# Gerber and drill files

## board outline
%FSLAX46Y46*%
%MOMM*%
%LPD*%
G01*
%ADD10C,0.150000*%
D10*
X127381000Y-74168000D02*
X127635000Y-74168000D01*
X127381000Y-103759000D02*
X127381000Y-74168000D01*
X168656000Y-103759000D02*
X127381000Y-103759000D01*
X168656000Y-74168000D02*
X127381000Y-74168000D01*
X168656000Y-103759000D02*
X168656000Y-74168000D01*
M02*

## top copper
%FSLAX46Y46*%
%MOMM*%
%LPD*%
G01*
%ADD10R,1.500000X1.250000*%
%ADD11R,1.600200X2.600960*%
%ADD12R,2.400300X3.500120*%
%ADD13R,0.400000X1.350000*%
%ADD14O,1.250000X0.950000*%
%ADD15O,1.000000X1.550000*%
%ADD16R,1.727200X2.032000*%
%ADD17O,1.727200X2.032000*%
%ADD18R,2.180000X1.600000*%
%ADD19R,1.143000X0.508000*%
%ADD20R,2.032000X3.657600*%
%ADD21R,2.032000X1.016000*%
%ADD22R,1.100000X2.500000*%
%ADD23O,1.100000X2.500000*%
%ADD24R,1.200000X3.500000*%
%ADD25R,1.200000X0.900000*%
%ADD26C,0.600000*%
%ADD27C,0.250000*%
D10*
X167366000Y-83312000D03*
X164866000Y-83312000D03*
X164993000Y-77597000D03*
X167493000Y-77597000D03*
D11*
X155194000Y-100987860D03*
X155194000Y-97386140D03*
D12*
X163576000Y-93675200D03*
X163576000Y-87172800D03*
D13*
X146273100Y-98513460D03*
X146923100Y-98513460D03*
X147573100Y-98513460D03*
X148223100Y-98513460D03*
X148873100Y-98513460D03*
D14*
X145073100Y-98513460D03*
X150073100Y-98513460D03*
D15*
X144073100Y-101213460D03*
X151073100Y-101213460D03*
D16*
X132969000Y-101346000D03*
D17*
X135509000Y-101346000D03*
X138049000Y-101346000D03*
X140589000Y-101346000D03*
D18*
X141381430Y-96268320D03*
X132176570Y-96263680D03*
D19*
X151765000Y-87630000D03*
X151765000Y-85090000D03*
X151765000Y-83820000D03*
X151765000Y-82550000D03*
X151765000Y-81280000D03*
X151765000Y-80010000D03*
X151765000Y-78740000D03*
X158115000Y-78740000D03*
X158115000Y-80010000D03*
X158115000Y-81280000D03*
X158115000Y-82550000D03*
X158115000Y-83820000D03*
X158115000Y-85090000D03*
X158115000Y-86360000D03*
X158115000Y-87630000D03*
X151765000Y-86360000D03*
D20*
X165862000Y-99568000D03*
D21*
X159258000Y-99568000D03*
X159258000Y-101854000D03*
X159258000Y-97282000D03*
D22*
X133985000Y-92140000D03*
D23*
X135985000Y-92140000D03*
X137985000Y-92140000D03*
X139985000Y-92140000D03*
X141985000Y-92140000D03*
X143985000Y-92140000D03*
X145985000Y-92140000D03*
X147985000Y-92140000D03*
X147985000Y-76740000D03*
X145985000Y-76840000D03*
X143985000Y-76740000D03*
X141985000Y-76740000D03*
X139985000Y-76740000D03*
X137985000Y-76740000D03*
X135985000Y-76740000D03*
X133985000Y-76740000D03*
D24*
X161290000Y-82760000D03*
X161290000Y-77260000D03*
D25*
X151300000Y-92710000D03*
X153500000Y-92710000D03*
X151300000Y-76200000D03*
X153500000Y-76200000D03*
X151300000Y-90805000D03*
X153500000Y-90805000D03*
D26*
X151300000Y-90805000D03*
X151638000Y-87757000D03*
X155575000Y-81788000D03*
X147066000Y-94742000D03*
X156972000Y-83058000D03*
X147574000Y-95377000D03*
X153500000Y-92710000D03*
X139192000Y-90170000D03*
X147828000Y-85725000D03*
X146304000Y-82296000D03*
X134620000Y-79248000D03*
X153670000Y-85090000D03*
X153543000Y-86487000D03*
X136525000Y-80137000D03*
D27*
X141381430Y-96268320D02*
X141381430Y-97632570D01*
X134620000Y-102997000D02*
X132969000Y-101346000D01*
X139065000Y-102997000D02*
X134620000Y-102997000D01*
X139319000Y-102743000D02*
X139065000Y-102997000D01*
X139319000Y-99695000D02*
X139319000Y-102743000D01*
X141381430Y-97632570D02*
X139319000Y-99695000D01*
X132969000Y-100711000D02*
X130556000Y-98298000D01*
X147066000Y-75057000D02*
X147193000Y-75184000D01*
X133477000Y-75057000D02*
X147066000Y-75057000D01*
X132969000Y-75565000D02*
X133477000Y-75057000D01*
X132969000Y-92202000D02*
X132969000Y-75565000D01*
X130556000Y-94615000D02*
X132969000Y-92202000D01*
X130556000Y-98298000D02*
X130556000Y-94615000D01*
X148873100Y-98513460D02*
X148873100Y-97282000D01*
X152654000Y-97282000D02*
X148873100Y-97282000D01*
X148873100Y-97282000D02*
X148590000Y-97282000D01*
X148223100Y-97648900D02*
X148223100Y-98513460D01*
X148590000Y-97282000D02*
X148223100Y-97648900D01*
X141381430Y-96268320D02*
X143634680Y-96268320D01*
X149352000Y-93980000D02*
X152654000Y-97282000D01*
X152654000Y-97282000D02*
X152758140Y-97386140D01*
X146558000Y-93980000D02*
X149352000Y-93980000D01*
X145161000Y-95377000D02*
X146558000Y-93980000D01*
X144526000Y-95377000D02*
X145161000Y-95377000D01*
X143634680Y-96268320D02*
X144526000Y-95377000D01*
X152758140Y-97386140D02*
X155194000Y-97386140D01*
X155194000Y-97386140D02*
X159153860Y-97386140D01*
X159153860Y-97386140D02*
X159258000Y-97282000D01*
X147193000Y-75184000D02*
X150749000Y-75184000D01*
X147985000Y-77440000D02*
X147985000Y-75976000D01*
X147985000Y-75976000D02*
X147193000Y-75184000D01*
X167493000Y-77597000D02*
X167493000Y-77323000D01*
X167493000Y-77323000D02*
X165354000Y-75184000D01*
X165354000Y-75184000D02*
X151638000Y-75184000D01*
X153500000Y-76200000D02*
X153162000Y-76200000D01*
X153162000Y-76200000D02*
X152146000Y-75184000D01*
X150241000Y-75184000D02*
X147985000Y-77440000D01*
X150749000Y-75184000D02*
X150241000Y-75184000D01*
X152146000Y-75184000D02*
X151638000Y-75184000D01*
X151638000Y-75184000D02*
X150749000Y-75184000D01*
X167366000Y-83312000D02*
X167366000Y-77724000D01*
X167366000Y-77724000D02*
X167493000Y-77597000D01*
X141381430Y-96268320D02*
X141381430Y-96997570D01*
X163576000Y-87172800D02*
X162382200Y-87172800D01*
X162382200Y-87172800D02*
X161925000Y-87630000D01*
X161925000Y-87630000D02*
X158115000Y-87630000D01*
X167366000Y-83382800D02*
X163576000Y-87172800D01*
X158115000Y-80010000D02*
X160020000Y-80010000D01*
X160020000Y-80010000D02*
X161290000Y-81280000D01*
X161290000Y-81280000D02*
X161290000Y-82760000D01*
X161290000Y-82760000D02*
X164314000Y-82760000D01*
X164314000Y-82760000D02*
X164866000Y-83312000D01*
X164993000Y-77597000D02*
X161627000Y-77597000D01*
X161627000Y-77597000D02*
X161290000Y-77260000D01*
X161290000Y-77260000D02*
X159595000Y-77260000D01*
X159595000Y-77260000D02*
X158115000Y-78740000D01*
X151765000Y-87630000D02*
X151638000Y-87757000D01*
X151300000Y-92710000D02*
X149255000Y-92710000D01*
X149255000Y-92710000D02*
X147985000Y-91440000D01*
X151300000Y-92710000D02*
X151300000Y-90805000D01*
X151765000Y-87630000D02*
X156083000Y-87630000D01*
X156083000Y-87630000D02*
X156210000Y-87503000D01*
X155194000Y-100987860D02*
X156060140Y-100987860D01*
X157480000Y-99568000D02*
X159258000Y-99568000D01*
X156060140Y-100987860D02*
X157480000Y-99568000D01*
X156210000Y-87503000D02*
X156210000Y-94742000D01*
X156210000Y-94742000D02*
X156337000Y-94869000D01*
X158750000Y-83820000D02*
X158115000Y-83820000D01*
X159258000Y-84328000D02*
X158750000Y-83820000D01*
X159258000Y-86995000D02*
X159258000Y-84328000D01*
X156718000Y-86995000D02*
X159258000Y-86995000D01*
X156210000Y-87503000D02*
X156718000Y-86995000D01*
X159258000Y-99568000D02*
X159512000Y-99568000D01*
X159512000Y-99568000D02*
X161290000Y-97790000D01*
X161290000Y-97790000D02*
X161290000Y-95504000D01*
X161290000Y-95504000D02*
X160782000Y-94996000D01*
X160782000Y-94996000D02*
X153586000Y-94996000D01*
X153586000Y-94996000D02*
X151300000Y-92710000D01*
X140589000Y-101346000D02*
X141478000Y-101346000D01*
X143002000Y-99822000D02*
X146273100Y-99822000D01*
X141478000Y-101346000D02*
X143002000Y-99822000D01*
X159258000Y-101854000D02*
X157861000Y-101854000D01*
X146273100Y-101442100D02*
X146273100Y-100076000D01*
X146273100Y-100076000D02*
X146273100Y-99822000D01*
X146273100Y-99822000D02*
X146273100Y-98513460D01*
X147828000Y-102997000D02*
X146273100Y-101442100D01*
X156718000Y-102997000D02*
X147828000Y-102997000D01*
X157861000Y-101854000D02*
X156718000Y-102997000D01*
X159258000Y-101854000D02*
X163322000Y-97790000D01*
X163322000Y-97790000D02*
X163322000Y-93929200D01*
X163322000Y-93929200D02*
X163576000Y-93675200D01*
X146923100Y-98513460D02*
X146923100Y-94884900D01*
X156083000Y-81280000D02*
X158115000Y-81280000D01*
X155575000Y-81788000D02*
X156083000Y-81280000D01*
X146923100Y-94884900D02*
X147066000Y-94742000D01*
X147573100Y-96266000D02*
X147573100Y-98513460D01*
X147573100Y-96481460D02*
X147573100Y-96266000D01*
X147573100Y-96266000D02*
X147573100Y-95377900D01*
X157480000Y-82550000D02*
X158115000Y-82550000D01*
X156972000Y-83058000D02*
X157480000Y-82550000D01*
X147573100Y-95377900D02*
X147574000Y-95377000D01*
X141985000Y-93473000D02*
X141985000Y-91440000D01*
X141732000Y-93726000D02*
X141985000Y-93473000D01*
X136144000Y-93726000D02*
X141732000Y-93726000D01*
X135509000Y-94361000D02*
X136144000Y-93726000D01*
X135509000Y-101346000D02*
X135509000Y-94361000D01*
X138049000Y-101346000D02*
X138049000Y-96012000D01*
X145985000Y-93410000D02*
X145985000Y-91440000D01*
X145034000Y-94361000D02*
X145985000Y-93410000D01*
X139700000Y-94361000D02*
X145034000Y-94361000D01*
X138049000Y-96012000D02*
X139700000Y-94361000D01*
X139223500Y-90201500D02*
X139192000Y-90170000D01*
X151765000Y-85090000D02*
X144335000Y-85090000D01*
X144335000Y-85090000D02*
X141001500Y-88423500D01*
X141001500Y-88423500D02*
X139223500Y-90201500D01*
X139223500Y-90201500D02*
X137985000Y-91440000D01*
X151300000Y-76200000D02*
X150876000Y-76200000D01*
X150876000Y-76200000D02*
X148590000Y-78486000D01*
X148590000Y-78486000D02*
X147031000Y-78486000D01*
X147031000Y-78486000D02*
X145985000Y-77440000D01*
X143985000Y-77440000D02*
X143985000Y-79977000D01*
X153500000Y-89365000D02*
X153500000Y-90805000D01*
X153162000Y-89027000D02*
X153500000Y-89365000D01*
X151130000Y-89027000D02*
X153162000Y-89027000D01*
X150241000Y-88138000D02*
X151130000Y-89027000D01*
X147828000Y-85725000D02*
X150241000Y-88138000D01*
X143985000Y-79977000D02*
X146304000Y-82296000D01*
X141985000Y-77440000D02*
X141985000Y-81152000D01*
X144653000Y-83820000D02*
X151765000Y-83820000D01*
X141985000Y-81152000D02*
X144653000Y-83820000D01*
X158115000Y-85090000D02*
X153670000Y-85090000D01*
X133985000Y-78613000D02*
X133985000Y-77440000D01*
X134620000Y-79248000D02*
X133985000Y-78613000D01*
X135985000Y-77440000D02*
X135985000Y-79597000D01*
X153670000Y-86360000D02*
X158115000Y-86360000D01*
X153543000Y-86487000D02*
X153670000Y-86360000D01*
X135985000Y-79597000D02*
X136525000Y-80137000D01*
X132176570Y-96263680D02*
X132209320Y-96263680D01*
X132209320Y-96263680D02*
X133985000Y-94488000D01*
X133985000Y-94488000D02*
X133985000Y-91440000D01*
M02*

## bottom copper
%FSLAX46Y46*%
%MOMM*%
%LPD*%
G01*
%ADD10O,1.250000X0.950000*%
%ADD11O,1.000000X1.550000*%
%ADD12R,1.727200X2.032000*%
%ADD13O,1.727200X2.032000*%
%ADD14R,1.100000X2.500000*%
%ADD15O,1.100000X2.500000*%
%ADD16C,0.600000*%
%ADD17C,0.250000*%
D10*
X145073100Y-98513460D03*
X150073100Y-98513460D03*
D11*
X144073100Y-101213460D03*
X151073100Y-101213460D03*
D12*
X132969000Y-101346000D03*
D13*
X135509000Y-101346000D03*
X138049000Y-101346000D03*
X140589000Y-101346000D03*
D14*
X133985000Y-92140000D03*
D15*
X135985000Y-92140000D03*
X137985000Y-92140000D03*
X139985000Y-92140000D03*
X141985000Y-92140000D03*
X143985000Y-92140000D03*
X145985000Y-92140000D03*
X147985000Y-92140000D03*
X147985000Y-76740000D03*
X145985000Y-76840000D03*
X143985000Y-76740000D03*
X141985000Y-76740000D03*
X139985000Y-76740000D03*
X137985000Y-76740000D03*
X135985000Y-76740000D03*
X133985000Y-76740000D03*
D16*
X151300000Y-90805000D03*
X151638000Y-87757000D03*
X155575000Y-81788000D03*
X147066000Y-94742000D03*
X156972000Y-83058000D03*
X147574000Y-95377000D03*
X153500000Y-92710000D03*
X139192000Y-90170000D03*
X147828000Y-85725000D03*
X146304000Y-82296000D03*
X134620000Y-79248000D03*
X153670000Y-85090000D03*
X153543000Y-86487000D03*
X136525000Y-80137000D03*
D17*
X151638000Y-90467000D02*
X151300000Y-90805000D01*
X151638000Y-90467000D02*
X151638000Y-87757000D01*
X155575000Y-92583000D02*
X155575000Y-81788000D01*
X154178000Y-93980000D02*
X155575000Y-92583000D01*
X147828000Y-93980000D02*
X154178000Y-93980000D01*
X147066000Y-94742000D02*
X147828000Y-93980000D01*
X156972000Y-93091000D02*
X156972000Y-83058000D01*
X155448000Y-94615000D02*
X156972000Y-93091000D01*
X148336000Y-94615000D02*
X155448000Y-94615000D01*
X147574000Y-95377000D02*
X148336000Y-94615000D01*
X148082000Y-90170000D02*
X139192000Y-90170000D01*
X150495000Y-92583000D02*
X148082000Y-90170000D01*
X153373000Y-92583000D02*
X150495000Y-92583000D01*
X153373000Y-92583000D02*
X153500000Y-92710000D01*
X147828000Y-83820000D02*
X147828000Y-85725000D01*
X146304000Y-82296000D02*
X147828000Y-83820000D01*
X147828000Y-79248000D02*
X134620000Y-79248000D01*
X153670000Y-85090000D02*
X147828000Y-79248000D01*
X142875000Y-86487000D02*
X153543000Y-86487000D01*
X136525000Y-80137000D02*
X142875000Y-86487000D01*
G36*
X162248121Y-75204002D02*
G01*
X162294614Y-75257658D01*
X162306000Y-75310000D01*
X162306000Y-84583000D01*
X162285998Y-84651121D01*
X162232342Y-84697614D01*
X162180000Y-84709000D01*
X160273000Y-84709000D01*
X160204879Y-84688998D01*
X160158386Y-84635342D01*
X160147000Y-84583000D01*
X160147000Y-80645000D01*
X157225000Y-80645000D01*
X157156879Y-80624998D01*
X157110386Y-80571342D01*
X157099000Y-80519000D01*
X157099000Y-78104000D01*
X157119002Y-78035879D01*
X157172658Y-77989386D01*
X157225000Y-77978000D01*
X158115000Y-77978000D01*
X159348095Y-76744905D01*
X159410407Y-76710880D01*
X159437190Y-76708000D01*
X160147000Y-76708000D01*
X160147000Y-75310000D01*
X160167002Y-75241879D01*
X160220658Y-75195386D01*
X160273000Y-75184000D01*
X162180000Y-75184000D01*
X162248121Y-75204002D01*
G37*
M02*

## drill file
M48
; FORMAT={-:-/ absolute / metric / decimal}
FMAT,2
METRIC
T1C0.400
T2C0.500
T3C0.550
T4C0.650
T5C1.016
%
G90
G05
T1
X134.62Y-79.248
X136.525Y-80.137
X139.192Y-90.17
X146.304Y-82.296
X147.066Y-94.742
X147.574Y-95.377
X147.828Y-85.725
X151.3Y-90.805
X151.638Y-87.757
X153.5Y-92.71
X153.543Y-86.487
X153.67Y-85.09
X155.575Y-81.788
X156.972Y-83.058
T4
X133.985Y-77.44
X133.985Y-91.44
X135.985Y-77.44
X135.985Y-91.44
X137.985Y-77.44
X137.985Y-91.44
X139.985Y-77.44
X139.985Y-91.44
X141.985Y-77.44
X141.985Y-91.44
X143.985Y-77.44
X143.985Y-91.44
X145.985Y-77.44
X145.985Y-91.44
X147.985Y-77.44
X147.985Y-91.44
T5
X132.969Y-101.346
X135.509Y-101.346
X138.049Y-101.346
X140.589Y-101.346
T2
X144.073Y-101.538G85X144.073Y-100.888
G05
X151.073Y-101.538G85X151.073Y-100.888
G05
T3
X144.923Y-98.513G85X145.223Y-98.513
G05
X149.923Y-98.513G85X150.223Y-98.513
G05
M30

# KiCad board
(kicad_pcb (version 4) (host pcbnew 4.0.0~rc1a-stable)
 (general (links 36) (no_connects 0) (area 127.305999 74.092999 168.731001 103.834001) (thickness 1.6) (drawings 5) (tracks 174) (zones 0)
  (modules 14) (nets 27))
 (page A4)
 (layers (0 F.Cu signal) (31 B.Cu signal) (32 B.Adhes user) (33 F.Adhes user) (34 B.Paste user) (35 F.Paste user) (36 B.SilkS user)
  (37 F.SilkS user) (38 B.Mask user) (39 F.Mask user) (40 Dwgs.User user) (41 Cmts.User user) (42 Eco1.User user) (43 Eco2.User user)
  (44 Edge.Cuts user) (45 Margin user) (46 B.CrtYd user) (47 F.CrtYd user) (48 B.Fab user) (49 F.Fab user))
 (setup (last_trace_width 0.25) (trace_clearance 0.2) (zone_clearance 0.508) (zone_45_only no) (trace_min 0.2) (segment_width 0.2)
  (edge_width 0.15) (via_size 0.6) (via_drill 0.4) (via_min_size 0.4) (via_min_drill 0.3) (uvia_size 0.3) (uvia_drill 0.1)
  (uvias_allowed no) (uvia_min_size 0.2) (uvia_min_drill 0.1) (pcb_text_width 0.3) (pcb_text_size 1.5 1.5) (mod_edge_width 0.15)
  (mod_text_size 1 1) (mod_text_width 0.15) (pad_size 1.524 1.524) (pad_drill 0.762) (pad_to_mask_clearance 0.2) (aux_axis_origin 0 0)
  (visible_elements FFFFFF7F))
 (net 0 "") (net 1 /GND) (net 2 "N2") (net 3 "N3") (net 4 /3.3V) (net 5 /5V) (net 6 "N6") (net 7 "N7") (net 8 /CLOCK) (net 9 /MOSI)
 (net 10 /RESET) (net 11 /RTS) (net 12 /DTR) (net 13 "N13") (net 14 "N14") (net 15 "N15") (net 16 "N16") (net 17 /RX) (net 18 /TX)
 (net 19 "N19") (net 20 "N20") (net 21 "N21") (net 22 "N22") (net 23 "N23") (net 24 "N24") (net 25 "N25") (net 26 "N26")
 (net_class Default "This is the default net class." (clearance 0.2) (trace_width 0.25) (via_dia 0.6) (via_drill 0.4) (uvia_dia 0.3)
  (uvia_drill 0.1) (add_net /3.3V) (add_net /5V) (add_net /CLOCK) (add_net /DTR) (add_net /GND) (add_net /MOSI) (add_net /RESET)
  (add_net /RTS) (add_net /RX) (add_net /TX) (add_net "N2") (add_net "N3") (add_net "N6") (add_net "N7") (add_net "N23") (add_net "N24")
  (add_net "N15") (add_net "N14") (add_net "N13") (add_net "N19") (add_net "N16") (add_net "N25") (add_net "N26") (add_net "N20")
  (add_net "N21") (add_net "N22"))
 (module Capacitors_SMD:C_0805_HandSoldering (layer F.Cu) (at 166.116 83.312 180)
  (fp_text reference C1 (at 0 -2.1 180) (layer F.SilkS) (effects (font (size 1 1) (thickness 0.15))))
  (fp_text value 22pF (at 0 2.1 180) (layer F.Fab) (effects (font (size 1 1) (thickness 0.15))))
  (pad 1 smd rect (at -1.25 0 180) (size 1.5 1.25) (layers F.Cu F.Paste F.Mask) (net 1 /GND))
  (pad 2 smd rect (at 1.25 0 180) (size 1.5 1.25) (layers F.Cu F.Paste F.Mask) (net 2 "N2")))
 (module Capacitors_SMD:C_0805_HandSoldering (layer F.Cu) (at 166.243 77.597)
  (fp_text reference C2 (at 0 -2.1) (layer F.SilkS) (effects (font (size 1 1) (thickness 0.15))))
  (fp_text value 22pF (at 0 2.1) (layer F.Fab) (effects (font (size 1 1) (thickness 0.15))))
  (pad 1 smd rect (at -1.25 0) (size 1.5 1.25) (layers F.Cu F.Paste F.Mask) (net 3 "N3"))
  (pad 2 smd rect (at 1.25 0) (size 1.5 1.25) (layers F.Cu F.Paste F.Mask) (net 1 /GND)))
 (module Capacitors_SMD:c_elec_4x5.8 (layer F.Cu) (at 155.194 99.187 270)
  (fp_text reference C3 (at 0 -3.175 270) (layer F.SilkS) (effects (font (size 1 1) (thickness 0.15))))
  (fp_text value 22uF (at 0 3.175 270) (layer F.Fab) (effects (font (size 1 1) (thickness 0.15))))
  (pad 1 smd rect (at 1.80086 0 270) (size 2.60096 1.6002) (layers F.Cu F.Paste F.Mask) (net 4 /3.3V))
  (pad 2 smd rect (at -1.80086 0 270) (size 2.60096 1.6002) (layers F.Cu F.Paste F.Mask) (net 1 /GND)))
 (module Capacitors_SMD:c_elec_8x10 (layer F.Cu) (at 163.576 90.424 270)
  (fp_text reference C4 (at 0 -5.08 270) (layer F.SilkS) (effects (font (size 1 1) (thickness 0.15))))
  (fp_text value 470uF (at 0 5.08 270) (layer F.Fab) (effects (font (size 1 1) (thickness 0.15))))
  (pad 1 smd rect (at 3.2512 0 270) (size 3.50012 2.4003) (layers F.Cu F.Paste F.Mask) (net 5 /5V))
  (pad 2 smd rect (at -3.2512 0 270) (size 3.50012 2.4003) (layers F.Cu F.Paste F.Mask) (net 1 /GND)))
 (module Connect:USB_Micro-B (layer F.Cu) (at 147.574 100.076)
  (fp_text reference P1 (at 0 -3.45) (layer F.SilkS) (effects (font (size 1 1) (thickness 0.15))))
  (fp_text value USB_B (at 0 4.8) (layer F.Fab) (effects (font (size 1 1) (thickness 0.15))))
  (pad 1 smd rect (at -1.3009 -1.56254 90) (size 1.35 0.4) (layers F.Cu F.Paste F.Mask) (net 5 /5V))
  (pad 2 smd rect (at -0.6509 -1.56254 90) (size 1.35 0.4) (layers F.Cu F.Paste F.Mask) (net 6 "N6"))
  (pad 3 smd rect (at -0.0009 -1.56254 90) (size 1.35 0.4) (layers F.Cu F.Paste F.Mask) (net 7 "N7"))
  (pad 4 smd rect (at 0.6491 -1.56254 90) (size 1.35 0.4) (layers F.Cu F.Paste F.Mask) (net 1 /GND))
  (pad 5 smd rect (at 1.2991 -1.56254 90) (size 1.35 0.4) (layers F.Cu F.Paste F.Mask) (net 1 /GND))
  (pad 6 thru_hole oval (at -2.5009 -1.56254 90) (size 0.95 1.25) (drill oval 0.55 0.85) (layers *.Cu *.Mask F.SilkS))
  (pad 6 thru_hole oval (at 2.4991 -1.56254 90) (size 0.95 1.25) (drill oval 0.55 0.85) (layers *.Cu *.Mask F.SilkS))
  (pad 6 thru_hole oval (at -3.5009 1.13746 90) (size 1.55 1) (drill oval 1.15 0.5) (layers *.Cu *.Mask F.SilkS))
  (pad 6 thru_hole oval (at 3.4991 1.13746 90) (size 1.55 1) (drill oval 1.15 0.5) (layers *.Cu *.Mask F.SilkS)))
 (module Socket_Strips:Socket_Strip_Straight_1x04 (layer F.Cu) (at 132.969 101.346)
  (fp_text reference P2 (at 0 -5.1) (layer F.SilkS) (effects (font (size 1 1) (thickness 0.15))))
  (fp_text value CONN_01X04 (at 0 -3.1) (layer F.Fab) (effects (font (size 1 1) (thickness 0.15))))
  (pad 1 thru_hole rect (at 0 0) (size 1.7272 2.032) (drill 1.016) (layers *.Cu *.Mask F.SilkS) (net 1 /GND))
  (pad 2 thru_hole oval (at 2.54 0) (size 1.7272 2.032) (drill 1.016) (layers *.Cu *.Mask F.SilkS) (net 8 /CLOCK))
  (pad 3 thru_hole oval (at 5.08 0) (size 1.7272 2.032) (drill 1.016) (layers *.Cu *.Mask F.SilkS) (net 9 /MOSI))
  (pad 4 thru_hole oval (at 7.62 0) (size 1.7272 2.032) (drill 1.016) (layers *.Cu *.Mask F.SilkS) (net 5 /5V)))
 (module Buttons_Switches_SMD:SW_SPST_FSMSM (layer F.Cu) (at 136.779 96.266 180)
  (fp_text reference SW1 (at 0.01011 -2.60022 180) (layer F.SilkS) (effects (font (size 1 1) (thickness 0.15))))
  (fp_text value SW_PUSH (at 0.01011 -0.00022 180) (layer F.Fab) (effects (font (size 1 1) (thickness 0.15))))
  (pad 1 smd rect (at -4.60243 -0.00232 180) (size 2.18 1.6) (layers F.Cu F.Paste F.Mask) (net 1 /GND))
  (pad 2 smd rect (at 4.60243 0.00232 180) (size 2.18 1.6) (layers F.Cu F.Paste F.Mask) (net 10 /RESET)))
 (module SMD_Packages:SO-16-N (layer F.Cu) (at 154.94 83.185 90)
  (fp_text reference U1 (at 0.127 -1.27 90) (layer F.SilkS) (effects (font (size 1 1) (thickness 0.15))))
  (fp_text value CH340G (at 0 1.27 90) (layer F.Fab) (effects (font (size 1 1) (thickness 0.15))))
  (pad 16 smd rect (at -4.445 -3.175 90) (size 0.508 1.143) (layers F.Cu F.Paste F.Mask) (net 4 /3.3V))
  (pad 14 smd rect (at -1.905 -3.175 90) (size 0.508 1.143) (layers F.Cu F.Paste F.Mask) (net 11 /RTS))
  (pad 13 smd rect (at -0.635 -3.175 90) (size 0.508 1.143) (layers F.Cu F.Paste F.Mask) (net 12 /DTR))
  (pad 12 smd rect (at 0.635 -3.175 90) (size 0.508 1.143) (layers F.Cu F.Paste F.Mask) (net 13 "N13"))
  (pad 11 smd rect (at 1.905 -3.175 90) (size 0.508 1.143) (layers F.Cu F.Paste F.Mask) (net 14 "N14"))
  (pad 10 smd rect (at 3.175 -3.175 90) (size 0.508 1.143) (layers F.Cu F.Paste F.Mask) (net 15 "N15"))
  (pad 9 smd rect (at 4.445 -3.175 90) (size 0.508 1.143) (layers F.Cu F.Paste F.Mask) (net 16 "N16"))
  (pad 8 smd rect (at 4.445 3.175 90) (size 0.508 1.143) (layers F.Cu F.Paste F.Mask) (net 3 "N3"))
  (pad 7 smd rect (at 3.175 3.175 90) (size 0.508 1.143) (layers F.Cu F.Paste F.Mask) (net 2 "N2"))
  (pad 6 smd rect (at 1.905 3.175 90) (size 0.508 1.143) (layers F.Cu F.Paste F.Mask) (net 6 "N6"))
  (pad 5 smd rect (at 0.635 3.175 90) (size 0.508 1.143) (layers F.Cu F.Paste F.Mask) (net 7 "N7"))
  (pad 4 smd rect (at -0.635 3.175 90) (size 0.508 1.143) (layers F.Cu F.Paste F.Mask) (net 4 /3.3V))
  (pad 3 smd rect (at -1.905 3.175 90) (size 0.508 1.143) (layers F.Cu F.Paste F.Mask) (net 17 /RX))
  (pad 2 smd rect (at -3.175 3.175 90) (size 0.508 1.143) (layers F.Cu F.Paste F.Mask) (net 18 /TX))
  (pad 1 smd rect (at -4.445 3.175 90) (size 0.508 1.143) (layers F.Cu F.Paste F.Mask) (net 1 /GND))
  (pad 15 smd rect (at -3.175 -3.175 90) (size 0.508 1.143) (layers F.Cu F.Paste F.Mask) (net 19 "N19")))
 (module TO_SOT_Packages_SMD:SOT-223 (layer F.Cu) (at 162.56 99.568 270)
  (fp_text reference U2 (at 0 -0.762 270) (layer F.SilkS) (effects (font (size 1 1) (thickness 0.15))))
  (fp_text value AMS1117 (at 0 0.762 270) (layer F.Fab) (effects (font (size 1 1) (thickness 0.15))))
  (pad 4 smd rect (at 0 -3.302 270) (size 3.6576 2.032) (layers F.Cu F.Paste F.Mask))
  (pad 2 smd rect (at 0 3.302 270) (size 1.016 2.032) (layers F.Cu F.Paste F.Mask) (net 4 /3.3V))
  (pad 3 smd rect (at 2.286 3.302 270) (size 1.016 2.032) (layers F.Cu F.Paste F.Mask) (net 5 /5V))
  (pad 1 smd rect (at -2.286 3.302 270) (size 1.016 2.032) (layers F.Cu F.Paste F.Mask) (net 1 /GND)))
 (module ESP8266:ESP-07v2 (layer F.Cu) (at 133.985 91.44 90)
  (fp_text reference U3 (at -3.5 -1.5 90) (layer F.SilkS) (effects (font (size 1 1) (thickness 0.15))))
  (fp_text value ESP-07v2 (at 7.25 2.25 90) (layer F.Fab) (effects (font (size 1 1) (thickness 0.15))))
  (pad 1 thru_hole rect (at 0 0 90) (size 2.5 1.1) (drill 0.65 (offset -0.7 0)) (layers *.Cu *.Mask F.SilkS) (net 10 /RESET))
  (pad 2 thru_hole oval (at 0 2 90) (size 2.5 1.1) (drill 0.65 (offset -0.7 0)) (layers *.Cu *.Mask F.SilkS) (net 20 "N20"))
  (pad 3 thru_hole oval (at 0 4 90) (size 2.5 1.1) (drill 0.65 (offset -0.7 0)) (layers *.Cu *.Mask F.SilkS) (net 11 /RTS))
  (pad 4 thru_hole oval (at 0 6 90) (size 2.5 1.1) (drill 0.65 (offset -0.7 0)) (layers *.Cu *.Mask F.SilkS) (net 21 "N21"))
  (pad 5 thru_hole oval (at 0 8 90) (size 2.5 1.1) (drill 0.65 (offset -0.7 0)) (layers *.Cu *.Mask F.SilkS) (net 8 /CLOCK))
  (pad 6 thru_hole oval (at 0 10 90) (size 2.5 1.1) (drill 0.65 (offset -0.7 0)) (layers *.Cu *.Mask F.SilkS) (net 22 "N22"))
  (pad 7 thru_hole oval (at 0 12 90) (size 2.5 1.1) (drill 0.65 (offset -0.7 0)) (layers *.Cu *.Mask F.SilkS) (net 9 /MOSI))
  (pad 8 thru_hole oval (at 0 14 90) (size 2.5 1.1) (drill 0.65 (offset -0.7 0)) (layers *.Cu *.Mask F.SilkS) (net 4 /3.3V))
  (pad 9 thru_hole oval (at 14 14 90) (size 2.5 1.1) (drill 0.65 (offset 0.7 0)) (layers *.Cu *.Mask F.SilkS) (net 1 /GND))
  (pad 10 thru_hole oval (at 14 12 90) (size 2.5 1.1) (drill 0.65 (offset 0.6 0)) (layers *.Cu *.Mask F.SilkS) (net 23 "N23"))
  (pad 11 thru_hole oval (at 14 10 90) (size 2.5 1.1) (drill 0.65 (offset 0.7 0)) (layers *.Cu *.Mask F.SilkS) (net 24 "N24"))
  (pad 12 thru_hole oval (at 14 8 90) (size 2.5 1.1) (drill 0.65 (offset 0.7 0)) (layers *.Cu *.Mask F.SilkS) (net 12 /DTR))
  (pad 13 thru_hole oval (at 14 6 90) (size 2.5 1.1) (drill 0.65 (offset 0.7 0)) (layers *.Cu *.Mask F.SilkS) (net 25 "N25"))
  (pad 14 thru_hole oval (at 14 4 90) (size 2.5 1.1) (drill 0.65 (offset 0.7 0)) (layers *.Cu *.Mask F.SilkS) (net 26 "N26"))
  (pad 15 thru_hole oval (at 14 2 90) (size 2.5 1.1) (drill 0.65 (offset 0.7 0)) (layers *.Cu *.Mask F.SilkS) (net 18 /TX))
  (pad 16 thru_hole oval (at 14 0 90) (size 2.5 1.1) (drill 0.65 (offset 0.7 0)) (layers *.Cu *.Mask F.SilkS) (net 17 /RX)))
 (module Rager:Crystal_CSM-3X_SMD (layer F.Cu) (at 161.29 80.01 90)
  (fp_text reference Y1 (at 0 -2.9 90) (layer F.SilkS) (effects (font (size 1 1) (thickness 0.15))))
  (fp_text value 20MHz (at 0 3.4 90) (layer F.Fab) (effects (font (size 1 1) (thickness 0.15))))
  (pad 1 smd rect (at -2.75 0 90) (size 3.5 1.2) (layers F.Cu F.Paste F.Mask) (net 2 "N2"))
  (pad 2 smd rect (at 2.75 0 90) (size 3.5 1.2) (layers F.Cu F.Paste F.Mask) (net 3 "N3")))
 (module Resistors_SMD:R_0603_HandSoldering (layer F.Cu) (at 152.4 92.71)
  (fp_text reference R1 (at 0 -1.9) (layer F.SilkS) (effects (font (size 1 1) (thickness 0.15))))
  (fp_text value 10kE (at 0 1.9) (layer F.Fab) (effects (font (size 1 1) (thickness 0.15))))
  (pad 1 smd rect (at -1.1 0) (size 1.2 0.9) (layers F.Cu F.Paste F.Mask) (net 4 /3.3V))
  (pad 2 smd rect (at 1.1 0) (size 1.2 0.9) (layers F.Cu F.Paste F.Mask) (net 11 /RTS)))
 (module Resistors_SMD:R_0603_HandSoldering (layer F.Cu) (at 152.4 76.2)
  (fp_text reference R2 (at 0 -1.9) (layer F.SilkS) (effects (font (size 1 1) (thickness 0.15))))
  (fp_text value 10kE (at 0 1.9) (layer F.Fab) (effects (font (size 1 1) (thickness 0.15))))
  (pad 1 smd rect (at -1.1 0) (size 1.2 0.9) (layers F.Cu F.Paste F.Mask) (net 23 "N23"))
  (pad 2 smd rect (at 1.1 0) (size 1.2 0.9) (layers F.Cu F.Paste F.Mask) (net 1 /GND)))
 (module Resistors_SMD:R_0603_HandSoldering (layer F.Cu) (at 152.4 90.805)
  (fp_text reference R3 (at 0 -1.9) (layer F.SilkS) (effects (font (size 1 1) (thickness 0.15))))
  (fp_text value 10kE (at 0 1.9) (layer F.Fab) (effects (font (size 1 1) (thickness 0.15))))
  (pad 1 smd rect (at -1.1 0) (size 1.2 0.9) (layers F.Cu F.Paste F.Mask) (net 4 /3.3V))
  (pad 2 smd rect (at 1.1 0) (size 1.2 0.9) (layers F.Cu F.Paste F.Mask) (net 24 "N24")))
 (gr_line (start 127.381 74.168) (end 127.635 74.168) (angle 90) (layer Edge.Cuts) (width 0.15))
 (gr_line (start 127.381 103.759) (end 127.381 74.168) (angle 90) (layer Edge.Cuts) (width 0.15))
 (gr_line (start 168.656 103.759) (end 127.381 103.759) (angle 90) (layer Edge.Cuts) (width 0.15))
 (gr_line (start 168.656 74.168) (end 127.381 74.168) (angle 90) (layer Edge.Cuts) (width 0.15))
 (gr_line (start 168.656 103.759) (end 168.656 74.168) (angle 90) (layer Edge.Cuts) (width 0.15))
 (segment (start 141.38143 96.26832) (end 141.38143 97.63257) (width 0.25) (layer F.Cu) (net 1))
 (segment (start 134.62 102.997) (end 132.969 101.346) (width 0.25) (layer F.Cu) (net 1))
 (segment (start 139.065 102.997) (end 134.62 102.997) (width 0.25) (layer F.Cu) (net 1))
 (segment (start 139.319 102.743) (end 139.065 102.997) (width 0.25) (layer F.Cu) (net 1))
 (segment (start 139.319 99.695) (end 139.319 102.743) (width 0.25) (layer F.Cu) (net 1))
 (segment (start 141.38143 97.63257) (end 139.319 99.695) (width 0.25) (layer F.Cu) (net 1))
 (segment (start 132.969 100.711) (end 130.556 98.298) (width 0.25) (layer F.Cu) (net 1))
 (segment (start 147.066 75.057) (end 147.193 75.184) (width 0.25) (layer F.Cu) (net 1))
 (segment (start 133.477 75.057) (end 147.066 75.057) (width 0.25) (layer F.Cu) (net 1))
 (segment (start 132.969 75.565) (end 133.477 75.057) (width 0.25) (layer F.Cu) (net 1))
 (segment (start 132.969 92.202) (end 132.969 75.565) (width 0.25) (layer F.Cu) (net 1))
 (segment (start 130.556 94.615) (end 132.969 92.202) (width 0.25) (layer F.Cu) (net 1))
 (segment (start 130.556 98.298) (end 130.556 94.615) (width 0.25) (layer F.Cu) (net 1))
 (segment (start 148.8731 98.51346) (end 148.8731 97.282) (width 0.25) (layer F.Cu) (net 1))
 (segment (start 152.654 97.282) (end 148.8731 97.282) (width 0.25) (layer F.Cu) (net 1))
 (segment (start 148.8731 97.282) (end 148.59 97.282) (width 0.25) (layer F.Cu) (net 1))
 (segment (start 148.2231 97.6489) (end 148.2231 98.51346) (width 0.25) (layer F.Cu) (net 1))
 (segment (start 148.59 97.282) (end 148.2231 97.6489) (width 0.25) (layer F.Cu) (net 1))
 (segment (start 141.38143 96.26832) (end 143.63468 96.26832) (width 0.25) (layer F.Cu) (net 1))
 (segment (start 149.352 93.98) (end 152.654 97.282) (width 0.25) (layer F.Cu) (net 1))
 (segment (start 152.654 97.282) (end 152.75814 97.38614) (width 0.25) (layer F.Cu) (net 1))
 (segment (start 146.558 93.98) (end 149.352 93.98) (width 0.25) (layer F.Cu) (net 1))
 (segment (start 145.161 95.377) (end 146.558 93.98) (width 0.25) (layer F.Cu) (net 1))
 (segment (start 144.526 95.377) (end 145.161 95.377) (width 0.25) (layer F.Cu) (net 1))
 (segment (start 143.63468 96.26832) (end 144.526 95.377) (width 0.25) (layer F.Cu) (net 1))
 (segment (start 152.75814 97.38614) (end 155.194 97.38614) (width 0.25) (layer F.Cu) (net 1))
 (segment (start 155.194 97.38614) (end 159.15386 97.38614) (width 0.25) (layer F.Cu) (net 1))
 (segment (start 159.15386 97.38614) (end 159.258 97.282) (width 0.25) (layer F.Cu) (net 1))
 (segment (start 147.193 75.184) (end 150.749 75.184) (width 0.25) (layer F.Cu) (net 1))
 (segment (start 147.985 77.44) (end 147.985 75.976) (width 0.25) (layer F.Cu) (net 1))
 (segment (start 147.985 75.976) (end 147.193 75.184) (width 0.25) (layer F.Cu) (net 1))
 (segment (start 167.493 77.597) (end 167.493 77.323) (width 0.25) (layer F.Cu) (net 1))
 (segment (start 167.493 77.323) (end 165.354 75.184) (width 0.25) (layer F.Cu) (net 1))
 (segment (start 165.354 75.184) (end 151.638 75.184) (width 0.25) (layer F.Cu) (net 1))
 (segment (start 153.5 76.2) (end 153.162 76.2) (width 0.25) (layer F.Cu) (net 1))
 (segment (start 153.162 76.2) (end 152.146 75.184) (width 0.25) (layer F.Cu) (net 1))
 (segment (start 150.241 75.184) (end 147.985 77.44) (width 0.25) (layer F.Cu) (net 1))
 (segment (start 150.749 75.184) (end 150.241 75.184) (width 0.25) (layer F.Cu) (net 1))
 (segment (start 152.146 75.184) (end 151.638 75.184) (width 0.25) (layer F.Cu) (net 1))
 (segment (start 151.638 75.184) (end 150.749 75.184) (width 0.25) (layer F.Cu) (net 1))
 (segment (start 167.366 83.312) (end 167.366 77.724) (width 0.25) (layer F.Cu) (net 1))
 (segment (start 167.366 77.724) (end 167.493 77.597) (width 0.25) (layer F.Cu) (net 1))
 (segment (start 141.38143 96.26832) (end 141.38143 96.99757) (width 0.25) (layer F.Cu) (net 1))
 (segment (start 163.576 87.1728) (end 162.3822 87.1728) (width 0.25) (layer F.Cu) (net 1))
 (segment (start 162.3822 87.1728) (end 161.925 87.63) (width 0.25) (layer F.Cu) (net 1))
 (segment (start 161.925 87.63) (end 158.115 87.63) (width 0.25) (layer F.Cu) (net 1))
 (segment (start 167.366 83.3828) (end 163.576 87.1728) (width 0.25) (layer F.Cu) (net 1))
 (segment (start 158.115 80.01) (end 160.02 80.01) (width 0.25) (layer F.Cu) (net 2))
 (segment (start 160.02 80.01) (end 161.29 81.28) (width 0.25) (layer F.Cu) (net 2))
 (segment (start 161.29 81.28) (end 161.29 82.76) (width 0.25) (layer F.Cu) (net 2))
 (segment (start 161.29 82.76) (end 164.314 82.76) (width 0.25) (layer F.Cu) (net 2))
 (segment (start 164.314 82.76) (end 164.866 83.312) (width 0.25) (layer F.Cu) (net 2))
 (segment (start 164.993 77.597) (end 161.627 77.597) (width 0.25) (layer F.Cu) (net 3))
 (segment (start 161.627 77.597) (end 161.29 77.26) (width 0.25) (layer F.Cu) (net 3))
 (segment (start 161.29 77.26) (end 159.595 77.26) (width 0.25) (layer F.Cu) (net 3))
 (segment (start 159.595 77.26) (end 158.115 78.74) (width 0.25) (layer F.Cu) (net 3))
 (via (at 151.3 90.805) (size 0.6) (drill 0.4) (layers F.Cu B.Cu) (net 4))
 (segment (start 151.638 90.467) (end 151.3 90.805) (width 0.25) (layer B.Cu) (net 4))
 (segment (start 151.638 90.467) (end 151.638 87.757) (width 0.25) (layer B.Cu) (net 4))
 (via (at 151.638 87.757) (size 0.6) (drill 0.4) (layers F.Cu B.Cu) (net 4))
 (segment (start 151.765 87.63) (end 151.638 87.757) (width 0.25) (layer F.Cu) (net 4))
 (segment (start 151.3 92.71) (end 149.255 92.71) (width 0.25) (layer F.Cu) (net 4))
 (segment (start 149.255 92.71) (end 147.985 91.44) (width 0.25) (layer F.Cu) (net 4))
 (segment (start 151.3 92.71) (end 151.3 90.805) (width 0.25) (layer F.Cu) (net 4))
 (segment (start 151.765 87.63) (end 156.083 87.63) (width 0.25) (layer F.Cu) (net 4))
 (segment (start 156.083 87.63) (end 156.21 87.503) (width 0.25) (layer F.Cu) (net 4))
 (segment (start 155.194 100.98786) (end 156.06014 100.98786) (width 0.25) (layer F.Cu) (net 4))
 (segment (start 157.48 99.568) (end 159.258 99.568) (width 0.25) (layer F.Cu) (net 4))
 (segment (start 156.06014 100.98786) (end 157.48 99.568) (width 0.25) (layer F.Cu) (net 4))
 (segment (start 156.21 87.503) (end 156.21 94.742) (width 0.25) (layer F.Cu) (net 4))
 (segment (start 156.21 94.742) (end 156.337 94.869) (width 0.25) (layer F.Cu) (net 4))
 (segment (start 158.75 83.82) (end 158.115 83.82) (width 0.25) (layer F.Cu) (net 4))
 (segment (start 159.258 84.328) (end 158.75 83.82) (width 0.25) (layer F.Cu) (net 4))
 (segment (start 159.258 86.995) (end 159.258 84.328) (width 0.25) (layer F.Cu) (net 4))
 (segment (start 156.718 86.995) (end 159.258 86.995) (width 0.25) (layer F.Cu) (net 4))
 (segment (start 156.21 87.503) (end 156.718 86.995) (width 0.25) (layer F.Cu) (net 4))
 (segment (start 159.258 99.568) (end 159.512 99.568) (width 0.25) (layer F.Cu) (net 4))
 (segment (start 159.512 99.568) (end 161.29 97.79) (width 0.25) (layer F.Cu) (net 4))
 (segment (start 161.29 97.79) (end 161.29 95.504) (width 0.25) (layer F.Cu) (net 4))
 (segment (start 161.29 95.504) (end 160.782 94.996) (width 0.25) (layer F.Cu) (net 4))
 (segment (start 160.782 94.996) (end 153.586 94.996) (width 0.25) (layer F.Cu) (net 4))
 (segment (start 153.586 94.996) (end 151.3 92.71) (width 0.25) (layer F.Cu) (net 4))
 (segment (start 140.589 101.346) (end 141.478 101.346) (width 0.25) (layer F.Cu) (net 5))
 (segment (start 143.002 99.822) (end 146.2731 99.822) (width 0.25) (layer F.Cu) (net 5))
 (segment (start 141.478 101.346) (end 143.002 99.822) (width 0.25) (layer F.Cu) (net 5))
 (segment (start 159.258 101.854) (end 157.861 101.854) (width 0.25) (layer F.Cu) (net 5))
 (segment (start 146.2731 101.4421) (end 146.2731 100.076) (width 0.25) (layer F.Cu) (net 5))
 (segment (start 146.2731 100.076) (end 146.2731 99.822) (width 0.25) (layer F.Cu) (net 5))
 (segment (start 146.2731 99.822) (end 146.2731 98.51346) (width 0.25) (layer F.Cu) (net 5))
 (segment (start 147.828 102.997) (end 146.2731 101.4421) (width 0.25) (layer F.Cu) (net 5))
 (segment (start 156.718 102.997) (end 147.828 102.997) (width 0.25) (layer F.Cu) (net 5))
 (segment (start 157.861 101.854) (end 156.718 102.997) (width 0.25) (layer F.Cu) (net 5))
 (segment (start 159.258 101.854) (end 163.322 97.79) (width 0.25) (layer F.Cu) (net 5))
 (segment (start 163.322 97.79) (end 163.322 93.9292) (width 0.25) (layer F.Cu) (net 5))
 (segment (start 163.322 93.9292) (end 163.576 93.6752) (width 0.25) (layer F.Cu) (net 5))
 (segment (start 146.9231 98.51346) (end 146.9231 94.8849) (width 0.25) (layer F.Cu) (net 6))
 (segment (start 156.083 81.28) (end 158.115 81.28) (width 0.25) (layer F.Cu) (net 6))
 (segment (start 155.575 81.788) (end 156.083 81.28) (width 0.25) (layer F.Cu) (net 6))
 (via (at 155.575 81.788) (size 0.6) (drill 0.4) (layers F.Cu B.Cu) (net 6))
 (segment (start 155.575 92.583) (end 155.575 81.788) (width 0.25) (layer B.Cu) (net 6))
 (segment (start 154.178 93.98) (end 155.575 92.583) (width 0.25) (layer B.Cu) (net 6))
 (segment (start 147.828 93.98) (end 154.178 93.98) (width 0.25) (layer B.Cu) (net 6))
 (segment (start 147.066 94.742) (end 147.828 93.98) (width 0.25) (layer B.Cu) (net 6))
 (via (at 147.066 94.742) (size 0.6) (drill 0.4) (layers F.Cu B.Cu) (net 6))
 (segment (start 146.9231 94.8849) (end 147.066 94.742) (width 0.25) (layer F.Cu) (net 6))
 (segment (start 147.5731 96.266) (end 147.5731 98.51346) (width 0.25) (layer F.Cu) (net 7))
 (segment (start 147.5731 96.48146) (end 147.5731 96.266) (width 0.25) (layer F.Cu) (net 7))
 (segment (start 147.5731 96.266) (end 147.5731 95.3779) (width 0.25) (layer F.Cu) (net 7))
 (segment (start 157.48 82.55) (end 158.115 82.55) (width 0.25) (layer F.Cu) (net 7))
 (segment (start 156.972 83.058) (end 157.48 82.55) (width 0.25) (layer F.Cu) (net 7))
 (via (at 156.972 83.058) (size 0.6) (drill 0.4) (layers F.Cu B.Cu) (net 7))
 (segment (start 156.972 93.091) (end 156.972 83.058) (width 0.25) (layer B.Cu) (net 7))
 (segment (start 155.448 94.615) (end 156.972 93.091) (width 0.25) (layer B.Cu) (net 7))
 (segment (start 148.336 94.615) (end 155.448 94.615) (width 0.25) (layer B.Cu) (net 7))
 (segment (start 147.574 95.377) (end 148.336 94.615) (width 0.25) (layer B.Cu) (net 7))
 (via (at 147.574 95.377) (size 0.6) (drill 0.4) (layers F.Cu B.Cu) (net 7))
 (segment (start 147.5731 95.3779) (end 147.574 95.377) (width 0.25) (layer F.Cu) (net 7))
 (segment (start 141.985 93.473) (end 141.985 91.44) (width 0.25) (layer F.Cu) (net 8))
 (segment (start 141.732 93.726) (end 141.985 93.473) (width 0.25) (layer F.Cu) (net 8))
 (segment (start 136.144 93.726) (end 141.732 93.726) (width 0.25) (layer F.Cu) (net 8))
 (segment (start 135.509 94.361) (end 136.144 93.726) (width 0.25) (layer F.Cu) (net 8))
 (segment (start 135.509 101.346) (end 135.509 94.361) (width 0.25) (layer F.Cu) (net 8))
 (segment (start 138.049 101.346) (end 138.049 96.012) (width 0.25) (layer F.Cu) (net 9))
 (segment (start 145.985 93.41) (end 145.985 91.44) (width 0.25) (layer F.Cu) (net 9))
 (segment (start 145.034 94.361) (end 145.985 93.41) (width 0.25) (layer F.Cu) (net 9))
 (segment (start 139.7 94.361) (end 145.034 94.361) (width 0.25) (layer F.Cu) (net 9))
 (segment (start 138.049 96.012) (end 139.7 94.361) (width 0.25) (layer F.Cu) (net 9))
 (via (at 153.5 92.71) (size 0.6) (drill 0.4) (layers F.Cu B.Cu) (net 11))
 (segment (start 139.2235 90.2015) (end 139.192 90.17) (width 0.25) (layer F.Cu) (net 11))
 (via (at 139.192 90.17) (size 0.6) (drill 0.4) (layers F.Cu B.Cu) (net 11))
 (segment (start 148.082 90.17) (end 139.192 90.17) (width 0.25) (layer B.Cu) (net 11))
 (segment (start 150.495 92.583) (end 148.082 90.17) (width 0.25) (layer B.Cu) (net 11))
 (segment (start 153.373 92.583) (end 150.495 92.583) (width 0.25) (layer B.Cu) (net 11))
 (segment (start 153.373 92.583) (end 153.5 92.71) (width 0.25) (layer B.Cu) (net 11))
 (segment (start 151.765 85.09) (end 144.335 85.09) (width 0.25) (layer F.Cu) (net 11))
 (segment (start 144.335 85.09) (end 141.0015 88.4235) (width 0.25) (layer F.Cu) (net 11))
 (segment (start 141.0015 88.4235) (end 139.2235 90.2015) (width 0.25) (layer F.Cu) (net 11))
 (segment (start 139.2235 90.2015) (end 137.985 91.44) (width 0.25) (layer F.Cu) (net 11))
 (segment (start 151.3 76.2) (end 150.876 76.2) (width 0.25) (layer F.Cu) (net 23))
 (segment (start 150.876 76.2) (end 148.59 78.486) (width 0.25) (layer F.Cu) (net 23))
 (segment (start 148.59 78.486) (end 147.031 78.486) (width 0.25) (layer F.Cu) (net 23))
 (segment (start 147.031 78.486) (end 145.985 77.44) (width 0.25) (layer F.Cu) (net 23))
 (segment (start 143.985 77.44) (end 143.985 79.977) (width 0.25) (layer F.Cu) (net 24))
 (segment (start 153.5 89.365) (end 153.5 90.805) (width 0.25) (layer F.Cu) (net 24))
 (segment (start 153.162 89.027) (end 153.5 89.365) (width 0.25) (layer F.Cu) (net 24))
 (segment (start 151.13 89.027) (end 153.162 89.027) (width 0.25) (layer F.Cu) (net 24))
 (segment (start 150.241 88.138) (end 151.13 89.027) (width 0.25) (layer F.Cu) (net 24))
 (segment (start 147.828 85.725) (end 150.241 88.138) (width 0.25) (layer F.Cu) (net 24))
 (via (at 147.828 85.725) (size 0.6) (drill 0.4) (layers F.Cu B.Cu) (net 24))
 (segment (start 147.828 83.82) (end 147.828 85.725) (width 0.25) (layer B.Cu) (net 24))
 (segment (start 146.304 82.296) (end 147.828 83.82) (width 0.25) (layer B.Cu) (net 24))
 (via (at 146.304 82.296) (size 0.6) (drill 0.4) (layers F.Cu B.Cu) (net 24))
 (segment (start 143.985 79.977) (end 146.304 82.296) (width 0.25) (layer F.Cu) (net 24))
 (segment (start 141.985 77.44) (end 141.985 81.152) (width 0.25) (layer F.Cu) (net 12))
 (segment (start 144.653 83.82) (end 151.765 83.82) (width 0.25) (layer F.Cu) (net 12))
 (segment (start 141.985 81.152) (end 144.653 83.82) (width 0.25) (layer F.Cu) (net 12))
 (segment (start 158.115 85.09) (end 153.67 85.09) (width 0.25) (layer F.Cu) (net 17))
 (segment (start 133.985 78.613) (end 133.985 77.44) (width 0.25) (layer F.Cu) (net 17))
 (segment (start 134.62 79.248) (end 133.985 78.613) (width 0.25) (layer F.Cu) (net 17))
 (via (at 134.62 79.248) (size 0.6) (drill 0.4) (layers F.Cu B.Cu) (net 17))
 (segment (start 147.828 79.248) (end 134.62 79.248) (width 0.25) (layer B.Cu) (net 17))
 (segment (start 153.67 85.09) (end 147.828 79.248) (width 0.25) (layer B.Cu) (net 17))
 (via (at 153.67 85.09) (size 0.6) (drill 0.4) (layers F.Cu B.Cu) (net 17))
 (segment (start 135.985 77.44) (end 135.985 79.597) (width 0.25) (layer F.Cu) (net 18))
 (segment (start 153.67 86.36) (end 158.115 86.36) (width 0.25) (layer F.Cu) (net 18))
 (segment (start 153.543 86.487) (end 153.67 86.36) (width 0.25) (layer F.Cu) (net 18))
 (via (at 153.543 86.487) (size 0.6) (drill 0.4) (layers F.Cu B.Cu) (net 18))
 (segment (start 142.875 86.487) (end 153.543 86.487) (width 0.25) (layer B.Cu) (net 18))
 (segment (start 136.525 80.137) (end 142.875 86.487) (width 0.25) (layer B.Cu) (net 18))
 (via (at 136.525 80.137) (size 0.6) (drill 0.4) (layers F.Cu B.Cu) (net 18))
 (segment (start 135.985 79.597) (end 136.525 80.137) (width 0.25) (layer F.Cu) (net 18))
 (segment (start 132.17657 96.26368) (end 132.20932 96.26368) (width 0.25) (layer F.Cu) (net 10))
 (segment (start 132.20932 96.26368) (end 133.985 94.488) (width 0.25) (layer F.Cu) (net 10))
 (segment (start 133.985 94.488) (end 133.985 91.44) (width 0.25) (layer F.Cu) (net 10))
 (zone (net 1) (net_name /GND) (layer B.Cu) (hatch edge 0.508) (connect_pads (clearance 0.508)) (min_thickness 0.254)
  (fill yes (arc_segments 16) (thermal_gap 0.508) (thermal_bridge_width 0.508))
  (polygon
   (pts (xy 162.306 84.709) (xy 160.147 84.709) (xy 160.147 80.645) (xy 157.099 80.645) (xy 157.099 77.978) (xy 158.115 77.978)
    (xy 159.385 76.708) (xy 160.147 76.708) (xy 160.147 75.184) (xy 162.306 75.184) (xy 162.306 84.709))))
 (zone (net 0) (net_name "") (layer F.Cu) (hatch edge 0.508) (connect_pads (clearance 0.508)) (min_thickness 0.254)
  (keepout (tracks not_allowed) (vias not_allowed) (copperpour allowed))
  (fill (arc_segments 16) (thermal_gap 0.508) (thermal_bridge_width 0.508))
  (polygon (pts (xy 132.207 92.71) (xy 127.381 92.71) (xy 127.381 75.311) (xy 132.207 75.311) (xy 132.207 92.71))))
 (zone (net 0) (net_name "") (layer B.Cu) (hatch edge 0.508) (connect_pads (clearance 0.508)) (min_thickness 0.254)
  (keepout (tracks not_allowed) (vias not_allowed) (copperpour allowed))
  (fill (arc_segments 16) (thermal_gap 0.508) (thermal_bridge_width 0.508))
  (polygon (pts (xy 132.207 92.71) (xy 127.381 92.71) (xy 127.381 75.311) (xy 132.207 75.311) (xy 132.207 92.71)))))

